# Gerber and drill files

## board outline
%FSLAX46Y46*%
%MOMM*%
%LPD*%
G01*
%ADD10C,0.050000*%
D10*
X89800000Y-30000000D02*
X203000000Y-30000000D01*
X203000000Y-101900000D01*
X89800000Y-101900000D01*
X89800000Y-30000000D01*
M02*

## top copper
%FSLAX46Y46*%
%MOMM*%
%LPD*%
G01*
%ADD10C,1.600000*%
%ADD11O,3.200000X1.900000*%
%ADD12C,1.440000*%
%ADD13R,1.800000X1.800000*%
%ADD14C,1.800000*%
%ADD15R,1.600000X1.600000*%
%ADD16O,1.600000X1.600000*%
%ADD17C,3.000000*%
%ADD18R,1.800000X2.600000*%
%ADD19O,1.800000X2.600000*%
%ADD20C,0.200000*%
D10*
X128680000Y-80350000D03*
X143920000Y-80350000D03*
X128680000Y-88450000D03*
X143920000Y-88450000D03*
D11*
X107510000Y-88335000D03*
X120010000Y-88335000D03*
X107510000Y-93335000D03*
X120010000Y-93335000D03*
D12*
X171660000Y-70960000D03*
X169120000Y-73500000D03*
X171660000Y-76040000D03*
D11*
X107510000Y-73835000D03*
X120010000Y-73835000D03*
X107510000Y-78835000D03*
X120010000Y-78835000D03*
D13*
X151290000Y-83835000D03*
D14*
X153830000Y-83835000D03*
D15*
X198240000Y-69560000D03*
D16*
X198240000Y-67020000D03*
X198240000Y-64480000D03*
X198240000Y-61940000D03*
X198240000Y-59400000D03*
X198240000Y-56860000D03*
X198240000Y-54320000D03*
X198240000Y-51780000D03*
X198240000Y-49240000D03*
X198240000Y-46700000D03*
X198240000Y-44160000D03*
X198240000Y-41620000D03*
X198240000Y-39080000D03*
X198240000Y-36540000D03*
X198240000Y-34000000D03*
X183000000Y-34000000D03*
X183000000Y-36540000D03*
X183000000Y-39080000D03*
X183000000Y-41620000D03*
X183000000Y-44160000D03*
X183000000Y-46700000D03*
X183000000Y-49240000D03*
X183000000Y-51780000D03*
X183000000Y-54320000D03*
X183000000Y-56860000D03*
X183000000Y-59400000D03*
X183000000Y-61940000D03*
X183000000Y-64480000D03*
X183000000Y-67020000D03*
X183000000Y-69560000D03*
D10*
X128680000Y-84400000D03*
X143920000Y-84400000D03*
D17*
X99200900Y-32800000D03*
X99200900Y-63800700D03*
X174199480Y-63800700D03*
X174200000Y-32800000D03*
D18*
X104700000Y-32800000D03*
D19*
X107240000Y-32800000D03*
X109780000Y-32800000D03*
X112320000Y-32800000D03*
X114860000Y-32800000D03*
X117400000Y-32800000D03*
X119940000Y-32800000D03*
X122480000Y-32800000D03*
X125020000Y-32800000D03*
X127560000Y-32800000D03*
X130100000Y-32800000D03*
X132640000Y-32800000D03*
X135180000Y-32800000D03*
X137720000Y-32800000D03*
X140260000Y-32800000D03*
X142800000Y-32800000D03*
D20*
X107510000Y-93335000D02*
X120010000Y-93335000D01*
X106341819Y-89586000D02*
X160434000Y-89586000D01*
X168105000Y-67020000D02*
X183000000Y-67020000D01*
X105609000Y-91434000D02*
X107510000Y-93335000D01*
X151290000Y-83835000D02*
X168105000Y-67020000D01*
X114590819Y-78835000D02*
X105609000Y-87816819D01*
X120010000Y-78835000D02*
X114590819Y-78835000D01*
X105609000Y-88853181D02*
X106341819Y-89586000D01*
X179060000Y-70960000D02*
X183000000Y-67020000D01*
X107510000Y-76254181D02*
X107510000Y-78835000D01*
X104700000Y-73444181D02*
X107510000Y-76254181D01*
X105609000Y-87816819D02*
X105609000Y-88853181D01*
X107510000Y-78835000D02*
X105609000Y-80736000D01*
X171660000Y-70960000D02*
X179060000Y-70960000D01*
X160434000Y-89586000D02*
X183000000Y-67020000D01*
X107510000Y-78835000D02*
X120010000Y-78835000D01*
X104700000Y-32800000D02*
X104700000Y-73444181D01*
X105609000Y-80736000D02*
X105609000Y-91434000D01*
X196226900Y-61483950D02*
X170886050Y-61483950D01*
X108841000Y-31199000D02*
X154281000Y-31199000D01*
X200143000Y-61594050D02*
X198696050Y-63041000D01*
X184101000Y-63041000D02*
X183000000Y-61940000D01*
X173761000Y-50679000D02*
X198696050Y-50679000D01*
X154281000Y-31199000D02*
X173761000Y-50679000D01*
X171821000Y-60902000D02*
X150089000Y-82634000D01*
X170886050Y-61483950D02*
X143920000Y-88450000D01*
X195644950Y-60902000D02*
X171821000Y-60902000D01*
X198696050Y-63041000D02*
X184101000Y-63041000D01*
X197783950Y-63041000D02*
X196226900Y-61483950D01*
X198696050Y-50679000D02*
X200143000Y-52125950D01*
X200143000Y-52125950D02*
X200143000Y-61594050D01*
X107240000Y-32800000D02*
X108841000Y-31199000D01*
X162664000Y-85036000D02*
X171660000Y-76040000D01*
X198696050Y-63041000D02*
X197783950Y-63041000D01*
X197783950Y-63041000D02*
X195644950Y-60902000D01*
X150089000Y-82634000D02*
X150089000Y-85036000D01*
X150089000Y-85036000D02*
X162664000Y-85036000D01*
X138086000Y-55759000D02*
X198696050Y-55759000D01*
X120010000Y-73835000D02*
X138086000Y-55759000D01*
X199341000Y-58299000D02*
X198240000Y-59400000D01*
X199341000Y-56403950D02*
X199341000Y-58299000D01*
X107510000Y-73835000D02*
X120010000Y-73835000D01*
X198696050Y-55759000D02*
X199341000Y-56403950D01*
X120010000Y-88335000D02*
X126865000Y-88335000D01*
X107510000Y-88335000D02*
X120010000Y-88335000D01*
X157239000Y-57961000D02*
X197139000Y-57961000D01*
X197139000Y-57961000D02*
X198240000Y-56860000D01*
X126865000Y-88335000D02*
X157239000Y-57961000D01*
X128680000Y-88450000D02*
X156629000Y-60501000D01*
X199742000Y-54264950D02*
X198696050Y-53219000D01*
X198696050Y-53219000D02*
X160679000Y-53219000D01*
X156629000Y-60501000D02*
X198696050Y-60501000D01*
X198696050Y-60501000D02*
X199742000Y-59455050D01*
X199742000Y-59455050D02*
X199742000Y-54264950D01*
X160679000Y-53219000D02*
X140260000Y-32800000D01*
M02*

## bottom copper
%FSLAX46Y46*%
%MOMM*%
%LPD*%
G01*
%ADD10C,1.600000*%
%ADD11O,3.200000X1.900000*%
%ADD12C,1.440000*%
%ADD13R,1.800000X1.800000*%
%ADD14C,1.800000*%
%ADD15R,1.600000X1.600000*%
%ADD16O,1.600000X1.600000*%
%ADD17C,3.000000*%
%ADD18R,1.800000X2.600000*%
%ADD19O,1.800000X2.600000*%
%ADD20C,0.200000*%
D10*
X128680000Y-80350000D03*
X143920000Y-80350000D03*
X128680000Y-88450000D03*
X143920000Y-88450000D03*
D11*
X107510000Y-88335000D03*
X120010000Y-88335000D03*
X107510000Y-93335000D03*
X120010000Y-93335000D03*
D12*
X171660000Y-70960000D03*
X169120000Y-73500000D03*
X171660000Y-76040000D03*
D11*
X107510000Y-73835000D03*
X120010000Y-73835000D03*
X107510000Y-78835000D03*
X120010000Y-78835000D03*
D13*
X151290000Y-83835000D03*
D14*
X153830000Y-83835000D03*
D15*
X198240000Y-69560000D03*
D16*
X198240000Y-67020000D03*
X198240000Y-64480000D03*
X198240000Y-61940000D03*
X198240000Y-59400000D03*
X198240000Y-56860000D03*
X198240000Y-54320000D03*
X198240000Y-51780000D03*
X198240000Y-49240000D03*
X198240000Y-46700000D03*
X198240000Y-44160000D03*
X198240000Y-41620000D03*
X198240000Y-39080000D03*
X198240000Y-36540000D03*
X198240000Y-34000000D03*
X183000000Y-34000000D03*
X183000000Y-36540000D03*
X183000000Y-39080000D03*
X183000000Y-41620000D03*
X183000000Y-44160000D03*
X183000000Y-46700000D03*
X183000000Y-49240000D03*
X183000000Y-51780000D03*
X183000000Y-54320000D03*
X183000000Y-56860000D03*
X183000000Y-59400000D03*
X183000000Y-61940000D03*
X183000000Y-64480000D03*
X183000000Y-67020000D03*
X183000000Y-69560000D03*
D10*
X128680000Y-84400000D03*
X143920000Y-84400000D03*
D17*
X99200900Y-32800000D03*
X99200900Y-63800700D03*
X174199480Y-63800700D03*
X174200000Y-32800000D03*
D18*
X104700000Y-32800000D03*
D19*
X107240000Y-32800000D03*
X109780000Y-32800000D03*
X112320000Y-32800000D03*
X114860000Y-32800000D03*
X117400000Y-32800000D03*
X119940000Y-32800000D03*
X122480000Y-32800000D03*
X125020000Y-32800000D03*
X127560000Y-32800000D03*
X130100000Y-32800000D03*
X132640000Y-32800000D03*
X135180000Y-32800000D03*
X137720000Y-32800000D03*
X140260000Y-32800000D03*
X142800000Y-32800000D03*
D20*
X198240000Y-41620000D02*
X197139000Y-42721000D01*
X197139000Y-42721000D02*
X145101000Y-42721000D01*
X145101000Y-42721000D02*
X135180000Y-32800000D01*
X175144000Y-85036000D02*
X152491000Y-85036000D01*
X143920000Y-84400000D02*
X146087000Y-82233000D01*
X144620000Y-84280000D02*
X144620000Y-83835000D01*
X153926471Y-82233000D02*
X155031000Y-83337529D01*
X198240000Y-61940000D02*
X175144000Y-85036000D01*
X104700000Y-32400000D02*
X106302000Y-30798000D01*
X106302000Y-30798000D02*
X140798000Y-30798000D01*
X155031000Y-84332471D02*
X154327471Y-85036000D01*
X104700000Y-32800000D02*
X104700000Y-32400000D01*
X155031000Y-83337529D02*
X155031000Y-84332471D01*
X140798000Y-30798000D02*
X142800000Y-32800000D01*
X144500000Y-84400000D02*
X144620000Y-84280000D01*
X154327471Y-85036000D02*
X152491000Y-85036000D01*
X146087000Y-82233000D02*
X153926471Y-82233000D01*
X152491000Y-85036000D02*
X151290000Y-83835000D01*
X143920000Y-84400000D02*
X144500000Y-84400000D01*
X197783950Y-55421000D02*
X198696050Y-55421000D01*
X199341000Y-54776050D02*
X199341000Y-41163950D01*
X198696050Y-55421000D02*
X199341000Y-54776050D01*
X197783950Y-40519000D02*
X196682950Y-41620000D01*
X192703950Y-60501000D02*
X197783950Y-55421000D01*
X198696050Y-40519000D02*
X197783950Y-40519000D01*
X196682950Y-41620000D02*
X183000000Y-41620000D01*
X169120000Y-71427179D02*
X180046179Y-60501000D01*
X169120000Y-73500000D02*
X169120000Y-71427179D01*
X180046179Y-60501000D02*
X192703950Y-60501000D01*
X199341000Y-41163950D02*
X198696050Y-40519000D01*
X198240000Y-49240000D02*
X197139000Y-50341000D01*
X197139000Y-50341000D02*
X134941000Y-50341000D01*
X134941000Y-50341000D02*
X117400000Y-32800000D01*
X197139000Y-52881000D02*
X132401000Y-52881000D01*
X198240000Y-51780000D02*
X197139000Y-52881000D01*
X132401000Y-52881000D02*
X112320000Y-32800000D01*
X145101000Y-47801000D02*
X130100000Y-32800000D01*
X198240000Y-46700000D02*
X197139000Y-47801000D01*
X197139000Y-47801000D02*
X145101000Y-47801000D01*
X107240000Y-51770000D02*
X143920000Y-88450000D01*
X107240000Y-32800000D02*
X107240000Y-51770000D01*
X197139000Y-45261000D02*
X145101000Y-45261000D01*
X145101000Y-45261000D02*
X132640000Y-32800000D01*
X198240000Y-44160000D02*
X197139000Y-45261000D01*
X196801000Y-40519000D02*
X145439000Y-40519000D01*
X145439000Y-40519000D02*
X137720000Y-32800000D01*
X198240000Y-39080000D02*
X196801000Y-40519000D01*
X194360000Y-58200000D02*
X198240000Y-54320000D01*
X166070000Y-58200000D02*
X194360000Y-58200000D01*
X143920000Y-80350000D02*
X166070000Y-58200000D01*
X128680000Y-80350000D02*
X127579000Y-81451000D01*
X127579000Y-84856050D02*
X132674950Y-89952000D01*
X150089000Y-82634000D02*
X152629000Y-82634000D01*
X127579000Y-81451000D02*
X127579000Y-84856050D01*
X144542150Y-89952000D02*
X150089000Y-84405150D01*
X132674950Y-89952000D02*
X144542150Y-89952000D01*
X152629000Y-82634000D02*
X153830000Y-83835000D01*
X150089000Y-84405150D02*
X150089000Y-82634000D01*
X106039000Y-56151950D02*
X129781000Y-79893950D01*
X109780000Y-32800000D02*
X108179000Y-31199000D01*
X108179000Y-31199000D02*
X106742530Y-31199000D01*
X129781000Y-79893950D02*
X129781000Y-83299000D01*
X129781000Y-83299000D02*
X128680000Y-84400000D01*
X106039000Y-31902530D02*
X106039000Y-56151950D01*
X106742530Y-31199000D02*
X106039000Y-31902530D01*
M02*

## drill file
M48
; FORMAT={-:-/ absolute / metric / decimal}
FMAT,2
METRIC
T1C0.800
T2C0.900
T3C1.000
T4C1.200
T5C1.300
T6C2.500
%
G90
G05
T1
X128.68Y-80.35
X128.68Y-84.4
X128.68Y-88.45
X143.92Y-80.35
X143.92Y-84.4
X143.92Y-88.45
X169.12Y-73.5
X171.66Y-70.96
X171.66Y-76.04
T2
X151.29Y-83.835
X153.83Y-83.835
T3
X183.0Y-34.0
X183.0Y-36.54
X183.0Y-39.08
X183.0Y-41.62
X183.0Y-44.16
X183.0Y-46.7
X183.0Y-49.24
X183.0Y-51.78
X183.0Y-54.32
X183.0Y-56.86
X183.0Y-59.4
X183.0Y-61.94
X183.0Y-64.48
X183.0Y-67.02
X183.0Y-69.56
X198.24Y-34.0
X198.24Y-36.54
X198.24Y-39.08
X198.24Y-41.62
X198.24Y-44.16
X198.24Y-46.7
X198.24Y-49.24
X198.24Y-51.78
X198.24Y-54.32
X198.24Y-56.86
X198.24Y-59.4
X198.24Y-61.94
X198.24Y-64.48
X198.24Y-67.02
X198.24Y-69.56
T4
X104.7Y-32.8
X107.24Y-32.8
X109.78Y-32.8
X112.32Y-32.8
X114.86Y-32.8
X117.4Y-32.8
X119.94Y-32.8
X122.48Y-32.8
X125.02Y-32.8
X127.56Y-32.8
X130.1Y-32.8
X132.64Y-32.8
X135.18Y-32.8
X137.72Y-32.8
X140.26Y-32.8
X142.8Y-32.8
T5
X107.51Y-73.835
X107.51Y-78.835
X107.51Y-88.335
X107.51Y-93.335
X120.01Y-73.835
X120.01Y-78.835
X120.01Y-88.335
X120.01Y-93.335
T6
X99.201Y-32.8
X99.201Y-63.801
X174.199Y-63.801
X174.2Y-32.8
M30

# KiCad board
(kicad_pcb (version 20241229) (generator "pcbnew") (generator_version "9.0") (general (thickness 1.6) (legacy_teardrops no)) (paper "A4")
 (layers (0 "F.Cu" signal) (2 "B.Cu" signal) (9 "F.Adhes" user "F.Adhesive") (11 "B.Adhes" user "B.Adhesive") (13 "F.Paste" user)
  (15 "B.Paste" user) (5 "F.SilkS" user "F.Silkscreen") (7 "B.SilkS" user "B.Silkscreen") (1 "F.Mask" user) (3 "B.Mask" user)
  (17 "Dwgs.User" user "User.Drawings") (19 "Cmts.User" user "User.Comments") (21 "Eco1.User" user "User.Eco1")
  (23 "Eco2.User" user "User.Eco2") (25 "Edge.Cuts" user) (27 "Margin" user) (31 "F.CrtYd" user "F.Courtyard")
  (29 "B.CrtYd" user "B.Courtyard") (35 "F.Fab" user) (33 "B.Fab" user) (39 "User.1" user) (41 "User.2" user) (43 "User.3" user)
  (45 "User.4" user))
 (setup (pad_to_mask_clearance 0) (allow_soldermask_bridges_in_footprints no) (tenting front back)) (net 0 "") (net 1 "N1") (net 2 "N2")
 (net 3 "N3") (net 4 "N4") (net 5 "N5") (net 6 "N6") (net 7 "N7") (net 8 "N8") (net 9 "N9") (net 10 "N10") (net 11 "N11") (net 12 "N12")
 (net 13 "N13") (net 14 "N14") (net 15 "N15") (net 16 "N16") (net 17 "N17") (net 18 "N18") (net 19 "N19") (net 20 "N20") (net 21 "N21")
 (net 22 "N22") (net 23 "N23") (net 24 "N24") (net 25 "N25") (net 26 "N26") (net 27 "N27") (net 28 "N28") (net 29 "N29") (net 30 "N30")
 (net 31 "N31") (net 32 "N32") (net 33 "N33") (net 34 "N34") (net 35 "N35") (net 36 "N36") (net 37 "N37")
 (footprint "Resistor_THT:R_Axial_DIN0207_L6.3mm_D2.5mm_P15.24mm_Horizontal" (layer "F.Cu") (at 128.68 80.35)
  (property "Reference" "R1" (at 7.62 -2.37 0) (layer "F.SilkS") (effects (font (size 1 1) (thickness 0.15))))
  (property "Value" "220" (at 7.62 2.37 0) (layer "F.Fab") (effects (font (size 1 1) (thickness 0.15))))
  (pad "1" thru_hole circle (at 0 0) (size 1.6 1.6) (drill 0.8) (layers "*.Cu" "*.Mask") (remove_unused_layers no) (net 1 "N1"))
  (pad "2" thru_hole circle (at 15.24 0) (size 1.6 1.6) (drill 0.8) (layers "*.Cu" "*.Mask") (remove_unused_layers no) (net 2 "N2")))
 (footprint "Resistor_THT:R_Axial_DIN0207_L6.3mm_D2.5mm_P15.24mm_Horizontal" (layer "F.Cu") (at 128.68 88.45)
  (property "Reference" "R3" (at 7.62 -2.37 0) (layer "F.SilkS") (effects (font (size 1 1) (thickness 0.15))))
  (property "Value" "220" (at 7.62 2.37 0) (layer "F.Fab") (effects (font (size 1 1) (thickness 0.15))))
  (pad "1" thru_hole circle (at 0 0) (size 1.6 1.6) (drill 0.8) (layers "*.Cu" "*.Mask") (remove_unused_layers no) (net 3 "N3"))
  (pad "2" thru_hole circle (at 15.24 0) (size 1.6 1.6) (drill 0.8) (layers "*.Cu" "*.Mask") (remove_unused_layers no) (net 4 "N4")))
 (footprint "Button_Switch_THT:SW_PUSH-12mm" (layer "F.Cu") (at 107.51 88.335)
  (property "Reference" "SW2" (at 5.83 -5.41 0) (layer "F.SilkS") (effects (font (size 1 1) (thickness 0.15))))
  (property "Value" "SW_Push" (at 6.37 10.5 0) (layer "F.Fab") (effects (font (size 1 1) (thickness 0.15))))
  (pad "1" thru_hole oval (at 0 0) (size 3.2 1.9) (drill 1.3) (layers "*.Cu" "*.Mask") (remove_unused_layers no) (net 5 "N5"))
  (pad "1" thru_hole oval (at 12.5 0) (size 3.2 1.9) (drill 1.3) (layers "*.Cu" "*.Mask") (remove_unused_layers no) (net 5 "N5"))
  (pad "2" thru_hole oval (at 0 5) (size 3.2 1.9) (drill 1.3) (layers "*.Cu" "*.Mask") (remove_unused_layers no) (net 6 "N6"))
  (pad "2" thru_hole oval (at 12.5 5) (size 3.2 1.9) (drill 1.3) (layers "*.Cu" "*.Mask") (remove_unused_layers no) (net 6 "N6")))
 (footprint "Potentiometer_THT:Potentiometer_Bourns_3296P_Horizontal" (layer "F.Cu") (at 171.66 70.96)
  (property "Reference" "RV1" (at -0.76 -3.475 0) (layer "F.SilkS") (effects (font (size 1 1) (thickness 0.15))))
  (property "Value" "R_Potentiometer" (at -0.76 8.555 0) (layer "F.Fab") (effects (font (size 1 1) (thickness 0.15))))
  (pad "1" thru_hole circle (at 0 0) (size 1.44 1.44) (drill 0.8) (layers "*.Cu" "*.Mask") (remove_unused_layers no) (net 6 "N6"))
  (pad "2" thru_hole circle (at -2.54 2.54) (size 1.44 1.44) (drill 0.8) (layers "*.Cu" "*.Mask") (remove_unused_layers no) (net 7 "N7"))
  (pad "3" thru_hole circle (at 0 5.08) (size 1.44 1.44) (drill 0.8) (layers "*.Cu" "*.Mask") (remove_unused_layers no) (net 4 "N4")))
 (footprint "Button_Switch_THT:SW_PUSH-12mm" (layer "F.Cu") (at 107.51 73.835)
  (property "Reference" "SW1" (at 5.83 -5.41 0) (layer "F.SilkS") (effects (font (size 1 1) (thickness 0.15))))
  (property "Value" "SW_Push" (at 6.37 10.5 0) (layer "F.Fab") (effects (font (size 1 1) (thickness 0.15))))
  (pad "1" thru_hole oval (at 0 0) (size 3.2 1.9) (drill 1.3) (layers "*.Cu" "*.Mask") (remove_unused_layers no) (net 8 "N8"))
  (pad "1" thru_hole oval (at 12.5 0) (size 3.2 1.9) (drill 1.3) (layers "*.Cu" "*.Mask") (remove_unused_layers no) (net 8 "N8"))
  (pad "2" thru_hole oval (at 0 5) (size 3.2 1.9) (drill 1.3) (layers "*.Cu" "*.Mask") (remove_unused_layers no) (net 6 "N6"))
  (pad "2" thru_hole oval (at 12.5 5) (size 3.2 1.9) (drill 1.3) (layers "*.Cu" "*.Mask") (remove_unused_layers no) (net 6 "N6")))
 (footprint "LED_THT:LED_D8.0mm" (layer "F.Cu") (at 151.29 83.835)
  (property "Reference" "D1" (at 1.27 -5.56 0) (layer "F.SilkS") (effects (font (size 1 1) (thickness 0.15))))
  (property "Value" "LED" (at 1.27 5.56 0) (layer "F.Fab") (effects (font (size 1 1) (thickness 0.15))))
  (pad "1" thru_hole rect (at 0 0) (size 1.8 1.8) (drill 0.9) (layers "*.Cu" "*.Mask") (remove_unused_layers no) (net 6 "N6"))
  (pad "2" thru_hole circle (at 2.54 0) (size 1.8 1.8) (drill 0.9) (layers "*.Cu" "*.Mask") (remove_unused_layers no) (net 1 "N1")))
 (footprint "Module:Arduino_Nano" (layer "F.Cu") (at 198.24 69.56 180)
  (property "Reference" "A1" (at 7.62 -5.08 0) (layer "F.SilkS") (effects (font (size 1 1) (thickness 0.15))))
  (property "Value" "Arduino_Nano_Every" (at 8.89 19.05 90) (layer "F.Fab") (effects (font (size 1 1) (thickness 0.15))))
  (pad "1" thru_hole rect (at 0 0 180) (size 1.6 1.6) (drill 1) (layers "*.Cu" "*.Mask") (remove_unused_layers no) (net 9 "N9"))
  (pad "2" thru_hole oval (at 0 2.54 180) (size 1.6 1.6) (drill 1) (layers "*.Cu" "*.Mask") (remove_unused_layers no) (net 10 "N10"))
  (pad "3" thru_hole oval (at 0 5.08 180) (size 1.6 1.6) (drill 1) (layers "*.Cu" "*.Mask") (remove_unused_layers no) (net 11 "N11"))
  (pad "4" thru_hole oval (at 0 7.62 180) (size 1.6 1.6) (drill 1) (layers "*.Cu" "*.Mask") (remove_unused_layers no) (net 6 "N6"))
  (pad "5" thru_hole oval (at 0 10.16 180) (size 1.6 1.6) (drill 1) (layers "*.Cu" "*.Mask") (remove_unused_layers no) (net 8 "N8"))
  (pad "6" thru_hole oval (at 0 12.7 180) (size 1.6 1.6) (drill 1) (layers "*.Cu" "*.Mask") (remove_unused_layers no) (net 5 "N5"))
  (pad "7" thru_hole oval (at 0 15.24 180) (size 1.6 1.6) (drill 1) (layers "*.Cu" "*.Mask") (remove_unused_layers no) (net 2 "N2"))
  (pad "8" thru_hole oval (at 0 17.78 180) (size 1.6 1.6) (drill 1) (layers "*.Cu" "*.Mask") (remove_unused_layers no) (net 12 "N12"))
  (pad "9" thru_hole oval (at 0 20.32 180) (size 1.6 1.6) (drill 1) (layers "*.Cu" "*.Mask") (remove_unused_layers no) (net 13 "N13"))
  (pad "10" thru_hole oval (at 0 22.86 180) (size 1.6 1.6) (drill 1) (layers "*.Cu" "*.Mask") (remove_unused_layers no) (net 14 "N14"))
  (pad "11" thru_hole oval (at 0 25.4 180) (size 1.6 1.6) (drill 1) (layers "*.Cu" "*.Mask") (remove_unused_layers no) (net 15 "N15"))
  (pad "12" thru_hole oval (at 0 27.94 180) (size 1.6 1.6) (drill 1) (layers "*.Cu" "*.Mask") (remove_unused_layers no) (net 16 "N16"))
  (pad "13" thru_hole oval (at 0 30.48 180) (size 1.6 1.6) (drill 1) (layers "*.Cu" "*.Mask") (remove_unused_layers no) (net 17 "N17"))
  (pad "14" thru_hole oval (at 0 33.02 180) (size 1.6 1.6) (drill 1) (layers "*.Cu" "*.Mask") (remove_unused_layers no) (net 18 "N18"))
  (pad "15" thru_hole oval (at 0 35.56 180) (size 1.6 1.6) (drill 1) (layers "*.Cu" "*.Mask") (remove_unused_layers no) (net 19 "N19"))
  (pad "16" thru_hole oval (at 15.24 35.56 180) (size 1.6 1.6) (drill 1) (layers "*.Cu" "*.Mask") (remove_unused_layers no) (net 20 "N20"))
  (pad "17" thru_hole oval (at 15.24 33.02 180) (size 1.6 1.6) (drill 1) (layers "*.Cu" "*.Mask") (remove_unused_layers no) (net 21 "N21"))
  (pad "18" thru_hole oval (at 15.24 30.48 180) (size 1.6 1.6) (drill 1) (layers "*.Cu" "*.Mask") (remove_unused_layers no) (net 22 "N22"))
  (pad "19" thru_hole oval (at 15.24 27.94 180) (size 1.6 1.6) (drill 1) (layers "*.Cu" "*.Mask") (remove_unused_layers no) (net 7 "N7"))
  (pad "20" thru_hole oval (at 15.24 25.4 180) (size 1.6 1.6) (drill 1) (layers "*.Cu" "*.Mask") (remove_unused_layers no) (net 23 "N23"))
  (pad "21" thru_hole oval (at 15.24 22.86 180) (size 1.6 1.6) (drill 1) (layers "*.Cu" "*.Mask") (remove_unused_layers no) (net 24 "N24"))
  (pad "22" thru_hole oval (at 15.24 20.32 180) (size 1.6 1.6) (drill 1) (layers "*.Cu" "*.Mask") (remove_unused_layers no) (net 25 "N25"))
  (pad "23" thru_hole oval (at 15.24 17.78 180) (size 1.6 1.6) (drill 1) (layers "*.Cu" "*.Mask") (remove_unused_layers no) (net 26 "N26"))
  (pad "24" thru_hole oval (at 15.24 15.24 180) (size 1.6 1.6) (drill 1) (layers "*.Cu" "*.Mask") (remove_unused_layers no) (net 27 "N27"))
  (pad "25" thru_hole oval (at 15.24 12.7 180) (size 1.6 1.6) (drill 1) (layers "*.Cu" "*.Mask") (remove_unused_layers no) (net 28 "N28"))
  (pad "26" thru_hole oval (at 15.24 10.16 180) (size 1.6 1.6) (drill 1) (layers "*.Cu" "*.Mask") (remove_unused_layers no) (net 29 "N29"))
  (pad "27" thru_hole oval (at 15.24 7.62 180) (size 1.6 1.6) (drill 1) (layers "*.Cu" "*.Mask") (remove_unused_layers no) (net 4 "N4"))
  (pad "28" thru_hole oval (at 15.24 5.08 180) (size 1.6 1.6) (drill 1) (layers "*.Cu" "*.Mask") (remove_unused_layers no) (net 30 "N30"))
  (pad "29" thru_hole oval (at 15.24 2.54 180) (size 1.6 1.6) (drill 1) (layers "*.Cu" "*.Mask") (remove_unused_layers no) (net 6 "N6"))
  (pad "30" thru_hole oval (at 15.24 0 180) (size 1.6 1.6) (drill 1) (layers "*.Cu" "*.Mask") (remove_unused_layers no) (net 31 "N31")))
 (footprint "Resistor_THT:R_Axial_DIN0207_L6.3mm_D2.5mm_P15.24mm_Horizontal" (layer "F.Cu") (at 128.68 84.4)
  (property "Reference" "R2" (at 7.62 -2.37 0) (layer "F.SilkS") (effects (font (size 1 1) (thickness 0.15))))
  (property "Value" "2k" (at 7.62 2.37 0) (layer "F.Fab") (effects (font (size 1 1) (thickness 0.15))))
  (pad "1" thru_hole circle (at 0 0) (size 1.6 1.6) (drill 0.8) (layers "*.Cu" "*.Mask") (remove_unused_layers no) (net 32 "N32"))
  (pad "2" thru_hole circle (at 15.24 0) (size 1.6 1.6) (drill 0.8) (layers "*.Cu" "*.Mask") (remove_unused_layers no) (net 6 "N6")))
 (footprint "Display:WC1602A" (layer "F.Cu") (at 104.7 32.8)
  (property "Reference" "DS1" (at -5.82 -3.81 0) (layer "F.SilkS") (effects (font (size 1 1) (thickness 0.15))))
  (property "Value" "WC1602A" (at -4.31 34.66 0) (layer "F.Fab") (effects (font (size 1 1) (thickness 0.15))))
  (pad "" thru_hole circle (at -5.4991 0) (size 3 3) (drill 2.5) (layers "*.Cu" "*.Mask") (remove_unused_layers no))
  (pad "" thru_hole circle (at -5.4991 31.0007) (size 3 3) (drill 2.5) (layers "*.Cu" "*.Mask") (remove_unused_layers no))
  (pad "" thru_hole circle (at 69.49948 31.0007) (size 3 3) (drill 2.5) (layers "*.Cu" "*.Mask") (remove_unused_layers no))
  (pad "" thru_hole circle (at 69.5 0) (size 3 3) (drill 2.5) (layers "*.Cu" "*.Mask") (remove_unused_layers no))
  (pad "1" thru_hole rect (at 0 0) (size 1.8 2.6) (drill 1.2) (layers "*.Cu" "*.Mask") (remove_unused_layers no) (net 6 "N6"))
  (pad "2" thru_hole oval (at 2.54 0) (size 1.8 2.6) (drill 1.2) (layers "*.Cu" "*.Mask") (remove_unused_layers no) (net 4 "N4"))
  (pad "3" thru_hole oval (at 5.08 0) (size 1.8 2.6) (drill 1.2) (layers "*.Cu" "*.Mask") (remove_unused_layers no) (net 32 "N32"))
  (pad "4" thru_hole oval (at 7.62 0) (size 1.8 2.6) (drill 1.2) (layers "*.Cu" "*.Mask") (remove_unused_layers no) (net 12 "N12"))
  (pad "5" thru_hole oval (at 10.16 0) (size 1.8 2.6) (drill 1.2) (layers "*.Cu" "*.Mask") (remove_unused_layers no) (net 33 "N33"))
  (pad "6" thru_hole oval (at 12.7 0) (size 1.8 2.6) (drill 1.2) (layers "*.Cu" "*.Mask") (remove_unused_layers no) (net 13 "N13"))
  (pad "7" thru_hole oval (at 15.24 0) (size 1.8 2.6) (drill 1.2) (layers "*.Cu" "*.Mask") (remove_unused_layers no) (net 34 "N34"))
  (pad "8" thru_hole oval (at 17.78 0) (size 1.8 2.6) (drill 1.2) (layers "*.Cu" "*.Mask") (remove_unused_layers no) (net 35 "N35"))
  (pad "9" thru_hole oval (at 20.32 0) (size 1.8 2.6) (drill 1.2) (layers "*.Cu" "*.Mask") (remove_unused_layers no) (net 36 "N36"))
  (pad "10" thru_hole oval (at 22.86 0) (size 1.8 2.6) (drill 1.2) (layers "*.Cu" "*.Mask") (remove_unused_layers no) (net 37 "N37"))
  (pad "11" thru_hole oval (at 25.4 0) (size 1.8 2.6) (drill 1.2) (layers "*.Cu" "*.Mask") (remove_unused_layers no) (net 14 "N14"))
  (pad "12" thru_hole oval (at 27.94 0) (size 1.8 2.6) (drill 1.2) (layers "*.Cu" "*.Mask") (remove_unused_layers no) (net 15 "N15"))
  (pad "13" thru_hole oval (at 30.48 0) (size 1.8 2.6) (drill 1.2) (layers "*.Cu" "*.Mask") (remove_unused_layers no) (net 16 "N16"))
  (pad "14" thru_hole oval (at 33.02 0) (size 1.8 2.6) (drill 1.2) (layers "*.Cu" "*.Mask") (remove_unused_layers no) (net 17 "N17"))
  (pad "15" thru_hole oval (at 35.56 0) (size 1.8 2.6) (drill 1.2) (layers "*.Cu" "*.Mask") (remove_unused_layers no) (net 3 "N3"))
  (pad "16" thru_hole oval (at 38.1 0) (size 1.8 2.6) (drill 1.2) (layers "*.Cu" "*.Mask") (remove_unused_layers no) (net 6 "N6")))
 (gr_rect (start 89.8 30) (end 203 101.9) (stroke (width 0.05) (type default)) (fill no) (layer "Edge.Cuts"))
 (segment (start 198.24 41.62) (end 197.139 42.721) (width 0.2) (layer "B.Cu") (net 16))
 (segment (start 197.139 42.721) (end 145.101 42.721) (width 0.2) (layer "B.Cu") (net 16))
 (segment (start 145.101 42.721) (end 135.18 32.8) (width 0.2) (layer "B.Cu") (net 16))
 (segment (start 107.51 93.335) (end 120.01 93.335) (width 0.2) (layer "F.Cu") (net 6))
 (segment (start 106.341819 89.586) (end 160.434 89.586) (width 0.2) (layer "F.Cu") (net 6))
 (segment (start 168.105 67.02) (end 183 67.02) (width 0.2) (layer "F.Cu") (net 6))
 (segment (start 105.609 91.434) (end 107.51 93.335) (width 0.2) (layer "F.Cu") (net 6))
 (segment (start 151.29 83.835) (end 168.105 67.02) (width 0.2) (layer "F.Cu") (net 6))
 (segment (start 114.590819 78.835) (end 105.609 87.816819) (width 0.2) (layer "F.Cu") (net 6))
 (segment (start 120.01 78.835) (end 114.590819 78.835) (width 0.2) (layer "F.Cu") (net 6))
 (segment (start 105.609 88.853181) (end 106.341819 89.586) (width 0.2) (layer "F.Cu") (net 6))
 (segment (start 179.06 70.96) (end 183 67.02) (width 0.2) (layer "F.Cu") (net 6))
 (segment (start 107.51 76.254181) (end 107.51 78.835) (width 0.2) (layer "F.Cu") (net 6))
 (segment (start 104.7 73.444181) (end 107.51 76.254181) (width 0.2) (layer "F.Cu") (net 6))
 (segment (start 105.609 87.816819) (end 105.609 88.853181) (width 0.2) (layer "F.Cu") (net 6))
 (segment (start 107.51 78.835) (end 105.609 80.736) (width 0.2) (layer "F.Cu") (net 6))
 (segment (start 171.66 70.96) (end 179.06 70.96) (width 0.2) (layer "F.Cu") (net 6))
 (segment (start 160.434 89.586) (end 183 67.02) (width 0.2) (layer "F.Cu") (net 6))
 (segment (start 107.51 78.835) (end 120.01 78.835) (width 0.2) (layer "F.Cu") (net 6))
 (segment (start 104.7 32.8) (end 104.7 73.444181) (width 0.2) (layer "F.Cu") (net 6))
 (segment (start 105.609 80.736) (end 105.609 91.434) (width 0.2) (layer "F.Cu") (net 6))
 (segment (start 175.144 85.036) (end 152.491 85.036) (width 0.2) (layer "B.Cu") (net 6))
 (segment (start 143.92 84.4) (end 146.087 82.233) (width 0.2) (layer "B.Cu") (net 6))
 (segment (start 144.62 84.28) (end 144.62 83.835) (width 0.2) (layer "B.Cu") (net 6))
 (segment (start 153.926471 82.233) (end 155.031 83.337529) (width 0.2) (layer "B.Cu") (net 6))
 (segment (start 198.24 61.94) (end 175.144 85.036) (width 0.2) (layer "B.Cu") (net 6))
 (segment (start 104.7 32.4) (end 106.302 30.798) (width 0.2) (layer "B.Cu") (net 6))
 (segment (start 106.302 30.798) (end 140.798 30.798) (width 0.2) (layer "B.Cu") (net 6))
 (segment (start 155.031 84.332471) (end 154.327471 85.036) (width 0.2) (layer "B.Cu") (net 6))
 (segment (start 104.7 32.8) (end 104.7 32.4) (width 0.2) (layer "B.Cu") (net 6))
 (segment (start 155.031 83.337529) (end 155.031 84.332471) (width 0.2) (layer "B.Cu") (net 6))
 (segment (start 140.798 30.798) (end 142.8 32.8) (width 0.2) (layer "B.Cu") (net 6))
 (segment (start 144.5 84.4) (end 144.62 84.28) (width 0.2) (layer "B.Cu") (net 6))
 (segment (start 154.327471 85.036) (end 152.491 85.036) (width 0.2) (layer "B.Cu") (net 6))
 (segment (start 146.087 82.233) (end 153.926471 82.233) (width 0.2) (layer "B.Cu") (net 6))
 (segment (start 152.491 85.036) (end 151.29 83.835) (width 0.2) (layer "B.Cu") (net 6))
 (segment (start 143.92 84.4) (end 144.5 84.4) (width 0.2) (layer "B.Cu") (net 6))
 (segment (start 197.78395 55.421) (end 198.69605 55.421) (width 0.2) (layer "B.Cu") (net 7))
 (segment (start 199.341 54.77605) (end 199.341 41.16395) (width 0.2) (layer "B.Cu") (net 7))
 (segment (start 198.69605 55.421) (end 199.341 54.77605) (width 0.2) (layer "B.Cu") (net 7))
 (segment (start 197.78395 40.519) (end 196.68295 41.62) (width 0.2) (layer "B.Cu") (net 7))
 (segment (start 192.70395 60.501) (end 197.78395 55.421) (width 0.2) (layer "B.Cu") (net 7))
 (segment (start 198.69605 40.519) (end 197.78395 40.519) (width 0.2) (layer "B.Cu") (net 7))
 (segment (start 196.68295 41.62) (end 183 41.62) (width 0.2) (layer "B.Cu") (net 7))
 (segment (start 169.12 71.427179) (end 180.046179 60.501) (width 0.2) (layer "B.Cu") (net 7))
 (segment (start 169.12 73.5) (end 169.12 71.427179) (width 0.2) (layer "B.Cu") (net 7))
 (segment (start 180.046179 60.501) (end 192.70395 60.501) (width 0.2) (layer "B.Cu") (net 7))
 (segment (start 199.341 41.16395) (end 198.69605 40.519) (width 0.2) (layer "B.Cu") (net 7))
 (segment (start 198.24 49.24) (end 197.139 50.341) (width 0.2) (layer "B.Cu") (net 13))
 (segment (start 197.139 50.341) (end 134.941 50.341) (width 0.2) (layer "B.Cu") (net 13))
 (segment (start 134.941 50.341) (end 117.4 32.8) (width 0.2) (layer "B.Cu") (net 13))
 (segment (start 197.139 52.881) (end 132.401 52.881) (width 0.2) (layer "B.Cu") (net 12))
 (segment (start 198.24 51.78) (end 197.139 52.881) (width 0.2) (layer "B.Cu") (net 12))
 (segment (start 132.401 52.881) (end 112.32 32.8) (width 0.2) (layer "B.Cu") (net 12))
 (segment (start 145.101 47.801) (end 130.1 32.8) (width 0.2) (layer "B.Cu") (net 14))
 (segment (start 198.24 46.7) (end 197.139 47.801) (width 0.2) (layer "B.Cu") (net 14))
 (segment (start 197.139 47.801) (end 145.101 47.801) (width 0.2) (layer "B.Cu") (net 14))
 (segment (start 196.2269 61.48395) (end 170.88605 61.48395) (width 0.2) (layer "F.Cu") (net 4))
 (segment (start 108.841 31.199) (end 154.281 31.199) (width 0.2) (layer "F.Cu") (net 4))
 (segment (start 200.143 61.59405) (end 198.69605 63.041) (width 0.2) (layer "F.Cu") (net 4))
 (segment (start 184.101 63.041) (end 183 61.94) (width 0.2) (layer "F.Cu") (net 4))
 (segment (start 173.761 50.679) (end 198.69605 50.679) (width 0.2) (layer "F.Cu") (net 4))
 (segment (start 154.281 31.199) (end 173.761 50.679) (width 0.2) (layer "F.Cu") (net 4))
 (segment (start 171.821 60.902) (end 150.089 82.634) (width 0.2) (layer "F.Cu") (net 4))
 (segment (start 170.88605 61.48395) (end 143.92 88.45) (width 0.2) (layer "F.Cu") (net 4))
 (segment (start 195.64495 60.902) (end 171.821 60.902) (width 0.2) (layer "F.Cu") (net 4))
 (segment (start 198.69605 63.041) (end 184.101 63.041) (width 0.2) (layer "F.Cu") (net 4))
 (segment (start 197.78395 63.041) (end 196.2269 61.48395) (width 0.2) (layer "F.Cu") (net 4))
 (segment (start 198.69605 50.679) (end 200.143 52.12595) (width 0.2) (layer "F.Cu") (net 4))
 (segment (start 200.143 52.12595) (end 200.143 61.59405) (width 0.2) (layer "F.Cu") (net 4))
 (segment (start 107.24 32.8) (end 108.841 31.199) (width 0.2) (layer "F.Cu") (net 4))
 (segment (start 162.664 85.036) (end 171.66 76.04) (width 0.2) (layer "F.Cu") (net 4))
 (segment (start 198.69605 63.041) (end 197.78395 63.041) (width 0.2) (layer "F.Cu") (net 4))
 (segment (start 197.78395 63.041) (end 195.64495 60.902) (width 0.2) (layer "F.Cu") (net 4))
 (segment (start 150.089 82.634) (end 150.089 85.036) (width 0.2) (layer "F.Cu") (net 4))
 (segment (start 150.089 85.036) (end 162.664 85.036) (width 0.2) (layer "F.Cu") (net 4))
 (segment (start 107.24 51.77) (end 143.92 88.45) (width 0.2) (layer "B.Cu") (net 4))
 (segment (start 107.24 32.8) (end 107.24 51.77) (width 0.2) (layer "B.Cu") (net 4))
 (segment (start 138.086 55.759) (end 198.69605 55.759) (width 0.2) (layer "F.Cu") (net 8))
 (segment (start 120.01 73.835) (end 138.086 55.759) (width 0.2) (layer "F.Cu") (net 8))
 (segment (start 199.341 58.299) (end 198.24 59.4) (width 0.2) (layer "F.Cu") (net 8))
 (segment (start 199.341 56.40395) (end 199.341 58.299) (width 0.2) (layer "F.Cu") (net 8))
 (segment (start 107.51 73.835) (end 120.01 73.835) (width 0.2) (layer "F.Cu") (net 8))
 (segment (start 198.69605 55.759) (end 199.341 56.40395) (width 0.2) (layer "F.Cu") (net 8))
 (segment (start 197.139 45.261) (end 145.101 45.261) (width 0.2) (layer "B.Cu") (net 15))
 (segment (start 145.101 45.261) (end 132.64 32.8) (width 0.2) (layer "B.Cu") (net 15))
 (segment (start 198.24 44.16) (end 197.139 45.261) (width 0.2) (layer "B.Cu") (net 15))
 (segment (start 196.801 40.519) (end 145.439 40.519) (width 0.2) (layer "B.Cu") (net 17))
 (segment (start 145.439 40.519) (end 137.72 32.8) (width 0.2) (layer "B.Cu") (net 17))
 (segment (start 198.24 39.08) (end 196.801 40.519) (width 0.2) (layer "B.Cu") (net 17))
 (segment (start 120.01 88.335) (end 126.865 88.335) (width 0.2) (layer "F.Cu") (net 5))
 (segment (start 107.51 88.335) (end 120.01 88.335) (width 0.2) (layer "F.Cu") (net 5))
 (segment (start 157.239 57.961) (end 197.139 57.961) (width 0.2) (layer "F.Cu") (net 5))
 (segment (start 197.139 57.961) (end 198.24 56.86) (width 0.2) (layer "F.Cu") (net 5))
 (segment (start 126.865 88.335) (end 157.239 57.961) (width 0.2) (layer "F.Cu") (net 5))
 (segment (start 194.36 58.2) (end 198.24 54.32) (width 0.2) (layer "B.Cu") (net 2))
 (segment (start 166.07 58.2) (end 194.36 58.2) (width 0.2) (layer "B.Cu") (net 2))
 (segment (start 143.92 80.35) (end 166.07 58.2) (width 0.2) (layer "B.Cu") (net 2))
 (segment (start 128.68 80.35) (end 127.579 81.451) (width 0.2) (layer "B.Cu") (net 1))
 (segment (start 127.579 84.85605) (end 132.67495 89.952) (width 0.2) (layer "B.Cu") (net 1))
 (segment (start 150.089 82.634) (end 152.629 82.634) (width 0.2) (layer "B.Cu") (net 1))
 (segment (start 127.579 81.451) (end 127.579 84.85605) (width 0.2) (layer "B.Cu") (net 1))
 (segment (start 144.54215 89.952) (end 150.089 84.40515) (width 0.2) (layer "B.Cu") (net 1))
 (segment (start 132.67495 89.952) (end 144.54215 89.952) (width 0.2) (layer "B.Cu") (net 1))
 (segment (start 152.629 82.634) (end 153.83 83.835) (width 0.2) (layer "B.Cu") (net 1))
 (segment (start 150.089 84.40515) (end 150.089 82.634) (width 0.2) (layer "B.Cu") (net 1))
 (segment (start 128.68 88.45) (end 156.629 60.501) (width 0.2) (layer "F.Cu") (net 3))
 (segment (start 199.742 54.26495) (end 198.69605 53.219) (width 0.2) (layer "F.Cu") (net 3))
 (segment (start 198.69605 53.219) (end 160.679 53.219) (width 0.2) (layer "F.Cu") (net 3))
 (segment (start 156.629 60.501) (end 198.69605 60.501) (width 0.2) (layer "F.Cu") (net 3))
 (segment (start 198.69605 60.501) (end 199.742 59.45505) (width 0.2) (layer "F.Cu") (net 3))
 (segment (start 199.742 59.45505) (end 199.742 54.26495) (width 0.2) (layer "F.Cu") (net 3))
 (segment (start 160.679 53.219) (end 140.26 32.8) (width 0.2) (layer "F.Cu") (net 3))
 (segment (start 106.039 56.15195) (end 129.781 79.89395) (width 0.2) (layer "B.Cu") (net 32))
 (segment (start 109.78 32.8) (end 108.179 31.199) (width 0.2) (layer "B.Cu") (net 32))
 (segment (start 108.179 31.199) (end 106.74253 31.199) (width 0.2) (layer "B.Cu") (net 32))
 (segment (start 129.781 79.89395) (end 129.781 83.299) (width 0.2) (layer "B.Cu") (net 32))
 (segment (start 129.781 83.299) (end 128.68 84.4) (width 0.2) (layer "B.Cu") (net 32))
 (segment (start 106.039 31.90253) (end 106.039 56.15195) (width 0.2) (layer "B.Cu") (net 32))
 (segment (start 106.74253 31.199) (end 106.039 31.90253) (width 0.2) (layer "B.Cu") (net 32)))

